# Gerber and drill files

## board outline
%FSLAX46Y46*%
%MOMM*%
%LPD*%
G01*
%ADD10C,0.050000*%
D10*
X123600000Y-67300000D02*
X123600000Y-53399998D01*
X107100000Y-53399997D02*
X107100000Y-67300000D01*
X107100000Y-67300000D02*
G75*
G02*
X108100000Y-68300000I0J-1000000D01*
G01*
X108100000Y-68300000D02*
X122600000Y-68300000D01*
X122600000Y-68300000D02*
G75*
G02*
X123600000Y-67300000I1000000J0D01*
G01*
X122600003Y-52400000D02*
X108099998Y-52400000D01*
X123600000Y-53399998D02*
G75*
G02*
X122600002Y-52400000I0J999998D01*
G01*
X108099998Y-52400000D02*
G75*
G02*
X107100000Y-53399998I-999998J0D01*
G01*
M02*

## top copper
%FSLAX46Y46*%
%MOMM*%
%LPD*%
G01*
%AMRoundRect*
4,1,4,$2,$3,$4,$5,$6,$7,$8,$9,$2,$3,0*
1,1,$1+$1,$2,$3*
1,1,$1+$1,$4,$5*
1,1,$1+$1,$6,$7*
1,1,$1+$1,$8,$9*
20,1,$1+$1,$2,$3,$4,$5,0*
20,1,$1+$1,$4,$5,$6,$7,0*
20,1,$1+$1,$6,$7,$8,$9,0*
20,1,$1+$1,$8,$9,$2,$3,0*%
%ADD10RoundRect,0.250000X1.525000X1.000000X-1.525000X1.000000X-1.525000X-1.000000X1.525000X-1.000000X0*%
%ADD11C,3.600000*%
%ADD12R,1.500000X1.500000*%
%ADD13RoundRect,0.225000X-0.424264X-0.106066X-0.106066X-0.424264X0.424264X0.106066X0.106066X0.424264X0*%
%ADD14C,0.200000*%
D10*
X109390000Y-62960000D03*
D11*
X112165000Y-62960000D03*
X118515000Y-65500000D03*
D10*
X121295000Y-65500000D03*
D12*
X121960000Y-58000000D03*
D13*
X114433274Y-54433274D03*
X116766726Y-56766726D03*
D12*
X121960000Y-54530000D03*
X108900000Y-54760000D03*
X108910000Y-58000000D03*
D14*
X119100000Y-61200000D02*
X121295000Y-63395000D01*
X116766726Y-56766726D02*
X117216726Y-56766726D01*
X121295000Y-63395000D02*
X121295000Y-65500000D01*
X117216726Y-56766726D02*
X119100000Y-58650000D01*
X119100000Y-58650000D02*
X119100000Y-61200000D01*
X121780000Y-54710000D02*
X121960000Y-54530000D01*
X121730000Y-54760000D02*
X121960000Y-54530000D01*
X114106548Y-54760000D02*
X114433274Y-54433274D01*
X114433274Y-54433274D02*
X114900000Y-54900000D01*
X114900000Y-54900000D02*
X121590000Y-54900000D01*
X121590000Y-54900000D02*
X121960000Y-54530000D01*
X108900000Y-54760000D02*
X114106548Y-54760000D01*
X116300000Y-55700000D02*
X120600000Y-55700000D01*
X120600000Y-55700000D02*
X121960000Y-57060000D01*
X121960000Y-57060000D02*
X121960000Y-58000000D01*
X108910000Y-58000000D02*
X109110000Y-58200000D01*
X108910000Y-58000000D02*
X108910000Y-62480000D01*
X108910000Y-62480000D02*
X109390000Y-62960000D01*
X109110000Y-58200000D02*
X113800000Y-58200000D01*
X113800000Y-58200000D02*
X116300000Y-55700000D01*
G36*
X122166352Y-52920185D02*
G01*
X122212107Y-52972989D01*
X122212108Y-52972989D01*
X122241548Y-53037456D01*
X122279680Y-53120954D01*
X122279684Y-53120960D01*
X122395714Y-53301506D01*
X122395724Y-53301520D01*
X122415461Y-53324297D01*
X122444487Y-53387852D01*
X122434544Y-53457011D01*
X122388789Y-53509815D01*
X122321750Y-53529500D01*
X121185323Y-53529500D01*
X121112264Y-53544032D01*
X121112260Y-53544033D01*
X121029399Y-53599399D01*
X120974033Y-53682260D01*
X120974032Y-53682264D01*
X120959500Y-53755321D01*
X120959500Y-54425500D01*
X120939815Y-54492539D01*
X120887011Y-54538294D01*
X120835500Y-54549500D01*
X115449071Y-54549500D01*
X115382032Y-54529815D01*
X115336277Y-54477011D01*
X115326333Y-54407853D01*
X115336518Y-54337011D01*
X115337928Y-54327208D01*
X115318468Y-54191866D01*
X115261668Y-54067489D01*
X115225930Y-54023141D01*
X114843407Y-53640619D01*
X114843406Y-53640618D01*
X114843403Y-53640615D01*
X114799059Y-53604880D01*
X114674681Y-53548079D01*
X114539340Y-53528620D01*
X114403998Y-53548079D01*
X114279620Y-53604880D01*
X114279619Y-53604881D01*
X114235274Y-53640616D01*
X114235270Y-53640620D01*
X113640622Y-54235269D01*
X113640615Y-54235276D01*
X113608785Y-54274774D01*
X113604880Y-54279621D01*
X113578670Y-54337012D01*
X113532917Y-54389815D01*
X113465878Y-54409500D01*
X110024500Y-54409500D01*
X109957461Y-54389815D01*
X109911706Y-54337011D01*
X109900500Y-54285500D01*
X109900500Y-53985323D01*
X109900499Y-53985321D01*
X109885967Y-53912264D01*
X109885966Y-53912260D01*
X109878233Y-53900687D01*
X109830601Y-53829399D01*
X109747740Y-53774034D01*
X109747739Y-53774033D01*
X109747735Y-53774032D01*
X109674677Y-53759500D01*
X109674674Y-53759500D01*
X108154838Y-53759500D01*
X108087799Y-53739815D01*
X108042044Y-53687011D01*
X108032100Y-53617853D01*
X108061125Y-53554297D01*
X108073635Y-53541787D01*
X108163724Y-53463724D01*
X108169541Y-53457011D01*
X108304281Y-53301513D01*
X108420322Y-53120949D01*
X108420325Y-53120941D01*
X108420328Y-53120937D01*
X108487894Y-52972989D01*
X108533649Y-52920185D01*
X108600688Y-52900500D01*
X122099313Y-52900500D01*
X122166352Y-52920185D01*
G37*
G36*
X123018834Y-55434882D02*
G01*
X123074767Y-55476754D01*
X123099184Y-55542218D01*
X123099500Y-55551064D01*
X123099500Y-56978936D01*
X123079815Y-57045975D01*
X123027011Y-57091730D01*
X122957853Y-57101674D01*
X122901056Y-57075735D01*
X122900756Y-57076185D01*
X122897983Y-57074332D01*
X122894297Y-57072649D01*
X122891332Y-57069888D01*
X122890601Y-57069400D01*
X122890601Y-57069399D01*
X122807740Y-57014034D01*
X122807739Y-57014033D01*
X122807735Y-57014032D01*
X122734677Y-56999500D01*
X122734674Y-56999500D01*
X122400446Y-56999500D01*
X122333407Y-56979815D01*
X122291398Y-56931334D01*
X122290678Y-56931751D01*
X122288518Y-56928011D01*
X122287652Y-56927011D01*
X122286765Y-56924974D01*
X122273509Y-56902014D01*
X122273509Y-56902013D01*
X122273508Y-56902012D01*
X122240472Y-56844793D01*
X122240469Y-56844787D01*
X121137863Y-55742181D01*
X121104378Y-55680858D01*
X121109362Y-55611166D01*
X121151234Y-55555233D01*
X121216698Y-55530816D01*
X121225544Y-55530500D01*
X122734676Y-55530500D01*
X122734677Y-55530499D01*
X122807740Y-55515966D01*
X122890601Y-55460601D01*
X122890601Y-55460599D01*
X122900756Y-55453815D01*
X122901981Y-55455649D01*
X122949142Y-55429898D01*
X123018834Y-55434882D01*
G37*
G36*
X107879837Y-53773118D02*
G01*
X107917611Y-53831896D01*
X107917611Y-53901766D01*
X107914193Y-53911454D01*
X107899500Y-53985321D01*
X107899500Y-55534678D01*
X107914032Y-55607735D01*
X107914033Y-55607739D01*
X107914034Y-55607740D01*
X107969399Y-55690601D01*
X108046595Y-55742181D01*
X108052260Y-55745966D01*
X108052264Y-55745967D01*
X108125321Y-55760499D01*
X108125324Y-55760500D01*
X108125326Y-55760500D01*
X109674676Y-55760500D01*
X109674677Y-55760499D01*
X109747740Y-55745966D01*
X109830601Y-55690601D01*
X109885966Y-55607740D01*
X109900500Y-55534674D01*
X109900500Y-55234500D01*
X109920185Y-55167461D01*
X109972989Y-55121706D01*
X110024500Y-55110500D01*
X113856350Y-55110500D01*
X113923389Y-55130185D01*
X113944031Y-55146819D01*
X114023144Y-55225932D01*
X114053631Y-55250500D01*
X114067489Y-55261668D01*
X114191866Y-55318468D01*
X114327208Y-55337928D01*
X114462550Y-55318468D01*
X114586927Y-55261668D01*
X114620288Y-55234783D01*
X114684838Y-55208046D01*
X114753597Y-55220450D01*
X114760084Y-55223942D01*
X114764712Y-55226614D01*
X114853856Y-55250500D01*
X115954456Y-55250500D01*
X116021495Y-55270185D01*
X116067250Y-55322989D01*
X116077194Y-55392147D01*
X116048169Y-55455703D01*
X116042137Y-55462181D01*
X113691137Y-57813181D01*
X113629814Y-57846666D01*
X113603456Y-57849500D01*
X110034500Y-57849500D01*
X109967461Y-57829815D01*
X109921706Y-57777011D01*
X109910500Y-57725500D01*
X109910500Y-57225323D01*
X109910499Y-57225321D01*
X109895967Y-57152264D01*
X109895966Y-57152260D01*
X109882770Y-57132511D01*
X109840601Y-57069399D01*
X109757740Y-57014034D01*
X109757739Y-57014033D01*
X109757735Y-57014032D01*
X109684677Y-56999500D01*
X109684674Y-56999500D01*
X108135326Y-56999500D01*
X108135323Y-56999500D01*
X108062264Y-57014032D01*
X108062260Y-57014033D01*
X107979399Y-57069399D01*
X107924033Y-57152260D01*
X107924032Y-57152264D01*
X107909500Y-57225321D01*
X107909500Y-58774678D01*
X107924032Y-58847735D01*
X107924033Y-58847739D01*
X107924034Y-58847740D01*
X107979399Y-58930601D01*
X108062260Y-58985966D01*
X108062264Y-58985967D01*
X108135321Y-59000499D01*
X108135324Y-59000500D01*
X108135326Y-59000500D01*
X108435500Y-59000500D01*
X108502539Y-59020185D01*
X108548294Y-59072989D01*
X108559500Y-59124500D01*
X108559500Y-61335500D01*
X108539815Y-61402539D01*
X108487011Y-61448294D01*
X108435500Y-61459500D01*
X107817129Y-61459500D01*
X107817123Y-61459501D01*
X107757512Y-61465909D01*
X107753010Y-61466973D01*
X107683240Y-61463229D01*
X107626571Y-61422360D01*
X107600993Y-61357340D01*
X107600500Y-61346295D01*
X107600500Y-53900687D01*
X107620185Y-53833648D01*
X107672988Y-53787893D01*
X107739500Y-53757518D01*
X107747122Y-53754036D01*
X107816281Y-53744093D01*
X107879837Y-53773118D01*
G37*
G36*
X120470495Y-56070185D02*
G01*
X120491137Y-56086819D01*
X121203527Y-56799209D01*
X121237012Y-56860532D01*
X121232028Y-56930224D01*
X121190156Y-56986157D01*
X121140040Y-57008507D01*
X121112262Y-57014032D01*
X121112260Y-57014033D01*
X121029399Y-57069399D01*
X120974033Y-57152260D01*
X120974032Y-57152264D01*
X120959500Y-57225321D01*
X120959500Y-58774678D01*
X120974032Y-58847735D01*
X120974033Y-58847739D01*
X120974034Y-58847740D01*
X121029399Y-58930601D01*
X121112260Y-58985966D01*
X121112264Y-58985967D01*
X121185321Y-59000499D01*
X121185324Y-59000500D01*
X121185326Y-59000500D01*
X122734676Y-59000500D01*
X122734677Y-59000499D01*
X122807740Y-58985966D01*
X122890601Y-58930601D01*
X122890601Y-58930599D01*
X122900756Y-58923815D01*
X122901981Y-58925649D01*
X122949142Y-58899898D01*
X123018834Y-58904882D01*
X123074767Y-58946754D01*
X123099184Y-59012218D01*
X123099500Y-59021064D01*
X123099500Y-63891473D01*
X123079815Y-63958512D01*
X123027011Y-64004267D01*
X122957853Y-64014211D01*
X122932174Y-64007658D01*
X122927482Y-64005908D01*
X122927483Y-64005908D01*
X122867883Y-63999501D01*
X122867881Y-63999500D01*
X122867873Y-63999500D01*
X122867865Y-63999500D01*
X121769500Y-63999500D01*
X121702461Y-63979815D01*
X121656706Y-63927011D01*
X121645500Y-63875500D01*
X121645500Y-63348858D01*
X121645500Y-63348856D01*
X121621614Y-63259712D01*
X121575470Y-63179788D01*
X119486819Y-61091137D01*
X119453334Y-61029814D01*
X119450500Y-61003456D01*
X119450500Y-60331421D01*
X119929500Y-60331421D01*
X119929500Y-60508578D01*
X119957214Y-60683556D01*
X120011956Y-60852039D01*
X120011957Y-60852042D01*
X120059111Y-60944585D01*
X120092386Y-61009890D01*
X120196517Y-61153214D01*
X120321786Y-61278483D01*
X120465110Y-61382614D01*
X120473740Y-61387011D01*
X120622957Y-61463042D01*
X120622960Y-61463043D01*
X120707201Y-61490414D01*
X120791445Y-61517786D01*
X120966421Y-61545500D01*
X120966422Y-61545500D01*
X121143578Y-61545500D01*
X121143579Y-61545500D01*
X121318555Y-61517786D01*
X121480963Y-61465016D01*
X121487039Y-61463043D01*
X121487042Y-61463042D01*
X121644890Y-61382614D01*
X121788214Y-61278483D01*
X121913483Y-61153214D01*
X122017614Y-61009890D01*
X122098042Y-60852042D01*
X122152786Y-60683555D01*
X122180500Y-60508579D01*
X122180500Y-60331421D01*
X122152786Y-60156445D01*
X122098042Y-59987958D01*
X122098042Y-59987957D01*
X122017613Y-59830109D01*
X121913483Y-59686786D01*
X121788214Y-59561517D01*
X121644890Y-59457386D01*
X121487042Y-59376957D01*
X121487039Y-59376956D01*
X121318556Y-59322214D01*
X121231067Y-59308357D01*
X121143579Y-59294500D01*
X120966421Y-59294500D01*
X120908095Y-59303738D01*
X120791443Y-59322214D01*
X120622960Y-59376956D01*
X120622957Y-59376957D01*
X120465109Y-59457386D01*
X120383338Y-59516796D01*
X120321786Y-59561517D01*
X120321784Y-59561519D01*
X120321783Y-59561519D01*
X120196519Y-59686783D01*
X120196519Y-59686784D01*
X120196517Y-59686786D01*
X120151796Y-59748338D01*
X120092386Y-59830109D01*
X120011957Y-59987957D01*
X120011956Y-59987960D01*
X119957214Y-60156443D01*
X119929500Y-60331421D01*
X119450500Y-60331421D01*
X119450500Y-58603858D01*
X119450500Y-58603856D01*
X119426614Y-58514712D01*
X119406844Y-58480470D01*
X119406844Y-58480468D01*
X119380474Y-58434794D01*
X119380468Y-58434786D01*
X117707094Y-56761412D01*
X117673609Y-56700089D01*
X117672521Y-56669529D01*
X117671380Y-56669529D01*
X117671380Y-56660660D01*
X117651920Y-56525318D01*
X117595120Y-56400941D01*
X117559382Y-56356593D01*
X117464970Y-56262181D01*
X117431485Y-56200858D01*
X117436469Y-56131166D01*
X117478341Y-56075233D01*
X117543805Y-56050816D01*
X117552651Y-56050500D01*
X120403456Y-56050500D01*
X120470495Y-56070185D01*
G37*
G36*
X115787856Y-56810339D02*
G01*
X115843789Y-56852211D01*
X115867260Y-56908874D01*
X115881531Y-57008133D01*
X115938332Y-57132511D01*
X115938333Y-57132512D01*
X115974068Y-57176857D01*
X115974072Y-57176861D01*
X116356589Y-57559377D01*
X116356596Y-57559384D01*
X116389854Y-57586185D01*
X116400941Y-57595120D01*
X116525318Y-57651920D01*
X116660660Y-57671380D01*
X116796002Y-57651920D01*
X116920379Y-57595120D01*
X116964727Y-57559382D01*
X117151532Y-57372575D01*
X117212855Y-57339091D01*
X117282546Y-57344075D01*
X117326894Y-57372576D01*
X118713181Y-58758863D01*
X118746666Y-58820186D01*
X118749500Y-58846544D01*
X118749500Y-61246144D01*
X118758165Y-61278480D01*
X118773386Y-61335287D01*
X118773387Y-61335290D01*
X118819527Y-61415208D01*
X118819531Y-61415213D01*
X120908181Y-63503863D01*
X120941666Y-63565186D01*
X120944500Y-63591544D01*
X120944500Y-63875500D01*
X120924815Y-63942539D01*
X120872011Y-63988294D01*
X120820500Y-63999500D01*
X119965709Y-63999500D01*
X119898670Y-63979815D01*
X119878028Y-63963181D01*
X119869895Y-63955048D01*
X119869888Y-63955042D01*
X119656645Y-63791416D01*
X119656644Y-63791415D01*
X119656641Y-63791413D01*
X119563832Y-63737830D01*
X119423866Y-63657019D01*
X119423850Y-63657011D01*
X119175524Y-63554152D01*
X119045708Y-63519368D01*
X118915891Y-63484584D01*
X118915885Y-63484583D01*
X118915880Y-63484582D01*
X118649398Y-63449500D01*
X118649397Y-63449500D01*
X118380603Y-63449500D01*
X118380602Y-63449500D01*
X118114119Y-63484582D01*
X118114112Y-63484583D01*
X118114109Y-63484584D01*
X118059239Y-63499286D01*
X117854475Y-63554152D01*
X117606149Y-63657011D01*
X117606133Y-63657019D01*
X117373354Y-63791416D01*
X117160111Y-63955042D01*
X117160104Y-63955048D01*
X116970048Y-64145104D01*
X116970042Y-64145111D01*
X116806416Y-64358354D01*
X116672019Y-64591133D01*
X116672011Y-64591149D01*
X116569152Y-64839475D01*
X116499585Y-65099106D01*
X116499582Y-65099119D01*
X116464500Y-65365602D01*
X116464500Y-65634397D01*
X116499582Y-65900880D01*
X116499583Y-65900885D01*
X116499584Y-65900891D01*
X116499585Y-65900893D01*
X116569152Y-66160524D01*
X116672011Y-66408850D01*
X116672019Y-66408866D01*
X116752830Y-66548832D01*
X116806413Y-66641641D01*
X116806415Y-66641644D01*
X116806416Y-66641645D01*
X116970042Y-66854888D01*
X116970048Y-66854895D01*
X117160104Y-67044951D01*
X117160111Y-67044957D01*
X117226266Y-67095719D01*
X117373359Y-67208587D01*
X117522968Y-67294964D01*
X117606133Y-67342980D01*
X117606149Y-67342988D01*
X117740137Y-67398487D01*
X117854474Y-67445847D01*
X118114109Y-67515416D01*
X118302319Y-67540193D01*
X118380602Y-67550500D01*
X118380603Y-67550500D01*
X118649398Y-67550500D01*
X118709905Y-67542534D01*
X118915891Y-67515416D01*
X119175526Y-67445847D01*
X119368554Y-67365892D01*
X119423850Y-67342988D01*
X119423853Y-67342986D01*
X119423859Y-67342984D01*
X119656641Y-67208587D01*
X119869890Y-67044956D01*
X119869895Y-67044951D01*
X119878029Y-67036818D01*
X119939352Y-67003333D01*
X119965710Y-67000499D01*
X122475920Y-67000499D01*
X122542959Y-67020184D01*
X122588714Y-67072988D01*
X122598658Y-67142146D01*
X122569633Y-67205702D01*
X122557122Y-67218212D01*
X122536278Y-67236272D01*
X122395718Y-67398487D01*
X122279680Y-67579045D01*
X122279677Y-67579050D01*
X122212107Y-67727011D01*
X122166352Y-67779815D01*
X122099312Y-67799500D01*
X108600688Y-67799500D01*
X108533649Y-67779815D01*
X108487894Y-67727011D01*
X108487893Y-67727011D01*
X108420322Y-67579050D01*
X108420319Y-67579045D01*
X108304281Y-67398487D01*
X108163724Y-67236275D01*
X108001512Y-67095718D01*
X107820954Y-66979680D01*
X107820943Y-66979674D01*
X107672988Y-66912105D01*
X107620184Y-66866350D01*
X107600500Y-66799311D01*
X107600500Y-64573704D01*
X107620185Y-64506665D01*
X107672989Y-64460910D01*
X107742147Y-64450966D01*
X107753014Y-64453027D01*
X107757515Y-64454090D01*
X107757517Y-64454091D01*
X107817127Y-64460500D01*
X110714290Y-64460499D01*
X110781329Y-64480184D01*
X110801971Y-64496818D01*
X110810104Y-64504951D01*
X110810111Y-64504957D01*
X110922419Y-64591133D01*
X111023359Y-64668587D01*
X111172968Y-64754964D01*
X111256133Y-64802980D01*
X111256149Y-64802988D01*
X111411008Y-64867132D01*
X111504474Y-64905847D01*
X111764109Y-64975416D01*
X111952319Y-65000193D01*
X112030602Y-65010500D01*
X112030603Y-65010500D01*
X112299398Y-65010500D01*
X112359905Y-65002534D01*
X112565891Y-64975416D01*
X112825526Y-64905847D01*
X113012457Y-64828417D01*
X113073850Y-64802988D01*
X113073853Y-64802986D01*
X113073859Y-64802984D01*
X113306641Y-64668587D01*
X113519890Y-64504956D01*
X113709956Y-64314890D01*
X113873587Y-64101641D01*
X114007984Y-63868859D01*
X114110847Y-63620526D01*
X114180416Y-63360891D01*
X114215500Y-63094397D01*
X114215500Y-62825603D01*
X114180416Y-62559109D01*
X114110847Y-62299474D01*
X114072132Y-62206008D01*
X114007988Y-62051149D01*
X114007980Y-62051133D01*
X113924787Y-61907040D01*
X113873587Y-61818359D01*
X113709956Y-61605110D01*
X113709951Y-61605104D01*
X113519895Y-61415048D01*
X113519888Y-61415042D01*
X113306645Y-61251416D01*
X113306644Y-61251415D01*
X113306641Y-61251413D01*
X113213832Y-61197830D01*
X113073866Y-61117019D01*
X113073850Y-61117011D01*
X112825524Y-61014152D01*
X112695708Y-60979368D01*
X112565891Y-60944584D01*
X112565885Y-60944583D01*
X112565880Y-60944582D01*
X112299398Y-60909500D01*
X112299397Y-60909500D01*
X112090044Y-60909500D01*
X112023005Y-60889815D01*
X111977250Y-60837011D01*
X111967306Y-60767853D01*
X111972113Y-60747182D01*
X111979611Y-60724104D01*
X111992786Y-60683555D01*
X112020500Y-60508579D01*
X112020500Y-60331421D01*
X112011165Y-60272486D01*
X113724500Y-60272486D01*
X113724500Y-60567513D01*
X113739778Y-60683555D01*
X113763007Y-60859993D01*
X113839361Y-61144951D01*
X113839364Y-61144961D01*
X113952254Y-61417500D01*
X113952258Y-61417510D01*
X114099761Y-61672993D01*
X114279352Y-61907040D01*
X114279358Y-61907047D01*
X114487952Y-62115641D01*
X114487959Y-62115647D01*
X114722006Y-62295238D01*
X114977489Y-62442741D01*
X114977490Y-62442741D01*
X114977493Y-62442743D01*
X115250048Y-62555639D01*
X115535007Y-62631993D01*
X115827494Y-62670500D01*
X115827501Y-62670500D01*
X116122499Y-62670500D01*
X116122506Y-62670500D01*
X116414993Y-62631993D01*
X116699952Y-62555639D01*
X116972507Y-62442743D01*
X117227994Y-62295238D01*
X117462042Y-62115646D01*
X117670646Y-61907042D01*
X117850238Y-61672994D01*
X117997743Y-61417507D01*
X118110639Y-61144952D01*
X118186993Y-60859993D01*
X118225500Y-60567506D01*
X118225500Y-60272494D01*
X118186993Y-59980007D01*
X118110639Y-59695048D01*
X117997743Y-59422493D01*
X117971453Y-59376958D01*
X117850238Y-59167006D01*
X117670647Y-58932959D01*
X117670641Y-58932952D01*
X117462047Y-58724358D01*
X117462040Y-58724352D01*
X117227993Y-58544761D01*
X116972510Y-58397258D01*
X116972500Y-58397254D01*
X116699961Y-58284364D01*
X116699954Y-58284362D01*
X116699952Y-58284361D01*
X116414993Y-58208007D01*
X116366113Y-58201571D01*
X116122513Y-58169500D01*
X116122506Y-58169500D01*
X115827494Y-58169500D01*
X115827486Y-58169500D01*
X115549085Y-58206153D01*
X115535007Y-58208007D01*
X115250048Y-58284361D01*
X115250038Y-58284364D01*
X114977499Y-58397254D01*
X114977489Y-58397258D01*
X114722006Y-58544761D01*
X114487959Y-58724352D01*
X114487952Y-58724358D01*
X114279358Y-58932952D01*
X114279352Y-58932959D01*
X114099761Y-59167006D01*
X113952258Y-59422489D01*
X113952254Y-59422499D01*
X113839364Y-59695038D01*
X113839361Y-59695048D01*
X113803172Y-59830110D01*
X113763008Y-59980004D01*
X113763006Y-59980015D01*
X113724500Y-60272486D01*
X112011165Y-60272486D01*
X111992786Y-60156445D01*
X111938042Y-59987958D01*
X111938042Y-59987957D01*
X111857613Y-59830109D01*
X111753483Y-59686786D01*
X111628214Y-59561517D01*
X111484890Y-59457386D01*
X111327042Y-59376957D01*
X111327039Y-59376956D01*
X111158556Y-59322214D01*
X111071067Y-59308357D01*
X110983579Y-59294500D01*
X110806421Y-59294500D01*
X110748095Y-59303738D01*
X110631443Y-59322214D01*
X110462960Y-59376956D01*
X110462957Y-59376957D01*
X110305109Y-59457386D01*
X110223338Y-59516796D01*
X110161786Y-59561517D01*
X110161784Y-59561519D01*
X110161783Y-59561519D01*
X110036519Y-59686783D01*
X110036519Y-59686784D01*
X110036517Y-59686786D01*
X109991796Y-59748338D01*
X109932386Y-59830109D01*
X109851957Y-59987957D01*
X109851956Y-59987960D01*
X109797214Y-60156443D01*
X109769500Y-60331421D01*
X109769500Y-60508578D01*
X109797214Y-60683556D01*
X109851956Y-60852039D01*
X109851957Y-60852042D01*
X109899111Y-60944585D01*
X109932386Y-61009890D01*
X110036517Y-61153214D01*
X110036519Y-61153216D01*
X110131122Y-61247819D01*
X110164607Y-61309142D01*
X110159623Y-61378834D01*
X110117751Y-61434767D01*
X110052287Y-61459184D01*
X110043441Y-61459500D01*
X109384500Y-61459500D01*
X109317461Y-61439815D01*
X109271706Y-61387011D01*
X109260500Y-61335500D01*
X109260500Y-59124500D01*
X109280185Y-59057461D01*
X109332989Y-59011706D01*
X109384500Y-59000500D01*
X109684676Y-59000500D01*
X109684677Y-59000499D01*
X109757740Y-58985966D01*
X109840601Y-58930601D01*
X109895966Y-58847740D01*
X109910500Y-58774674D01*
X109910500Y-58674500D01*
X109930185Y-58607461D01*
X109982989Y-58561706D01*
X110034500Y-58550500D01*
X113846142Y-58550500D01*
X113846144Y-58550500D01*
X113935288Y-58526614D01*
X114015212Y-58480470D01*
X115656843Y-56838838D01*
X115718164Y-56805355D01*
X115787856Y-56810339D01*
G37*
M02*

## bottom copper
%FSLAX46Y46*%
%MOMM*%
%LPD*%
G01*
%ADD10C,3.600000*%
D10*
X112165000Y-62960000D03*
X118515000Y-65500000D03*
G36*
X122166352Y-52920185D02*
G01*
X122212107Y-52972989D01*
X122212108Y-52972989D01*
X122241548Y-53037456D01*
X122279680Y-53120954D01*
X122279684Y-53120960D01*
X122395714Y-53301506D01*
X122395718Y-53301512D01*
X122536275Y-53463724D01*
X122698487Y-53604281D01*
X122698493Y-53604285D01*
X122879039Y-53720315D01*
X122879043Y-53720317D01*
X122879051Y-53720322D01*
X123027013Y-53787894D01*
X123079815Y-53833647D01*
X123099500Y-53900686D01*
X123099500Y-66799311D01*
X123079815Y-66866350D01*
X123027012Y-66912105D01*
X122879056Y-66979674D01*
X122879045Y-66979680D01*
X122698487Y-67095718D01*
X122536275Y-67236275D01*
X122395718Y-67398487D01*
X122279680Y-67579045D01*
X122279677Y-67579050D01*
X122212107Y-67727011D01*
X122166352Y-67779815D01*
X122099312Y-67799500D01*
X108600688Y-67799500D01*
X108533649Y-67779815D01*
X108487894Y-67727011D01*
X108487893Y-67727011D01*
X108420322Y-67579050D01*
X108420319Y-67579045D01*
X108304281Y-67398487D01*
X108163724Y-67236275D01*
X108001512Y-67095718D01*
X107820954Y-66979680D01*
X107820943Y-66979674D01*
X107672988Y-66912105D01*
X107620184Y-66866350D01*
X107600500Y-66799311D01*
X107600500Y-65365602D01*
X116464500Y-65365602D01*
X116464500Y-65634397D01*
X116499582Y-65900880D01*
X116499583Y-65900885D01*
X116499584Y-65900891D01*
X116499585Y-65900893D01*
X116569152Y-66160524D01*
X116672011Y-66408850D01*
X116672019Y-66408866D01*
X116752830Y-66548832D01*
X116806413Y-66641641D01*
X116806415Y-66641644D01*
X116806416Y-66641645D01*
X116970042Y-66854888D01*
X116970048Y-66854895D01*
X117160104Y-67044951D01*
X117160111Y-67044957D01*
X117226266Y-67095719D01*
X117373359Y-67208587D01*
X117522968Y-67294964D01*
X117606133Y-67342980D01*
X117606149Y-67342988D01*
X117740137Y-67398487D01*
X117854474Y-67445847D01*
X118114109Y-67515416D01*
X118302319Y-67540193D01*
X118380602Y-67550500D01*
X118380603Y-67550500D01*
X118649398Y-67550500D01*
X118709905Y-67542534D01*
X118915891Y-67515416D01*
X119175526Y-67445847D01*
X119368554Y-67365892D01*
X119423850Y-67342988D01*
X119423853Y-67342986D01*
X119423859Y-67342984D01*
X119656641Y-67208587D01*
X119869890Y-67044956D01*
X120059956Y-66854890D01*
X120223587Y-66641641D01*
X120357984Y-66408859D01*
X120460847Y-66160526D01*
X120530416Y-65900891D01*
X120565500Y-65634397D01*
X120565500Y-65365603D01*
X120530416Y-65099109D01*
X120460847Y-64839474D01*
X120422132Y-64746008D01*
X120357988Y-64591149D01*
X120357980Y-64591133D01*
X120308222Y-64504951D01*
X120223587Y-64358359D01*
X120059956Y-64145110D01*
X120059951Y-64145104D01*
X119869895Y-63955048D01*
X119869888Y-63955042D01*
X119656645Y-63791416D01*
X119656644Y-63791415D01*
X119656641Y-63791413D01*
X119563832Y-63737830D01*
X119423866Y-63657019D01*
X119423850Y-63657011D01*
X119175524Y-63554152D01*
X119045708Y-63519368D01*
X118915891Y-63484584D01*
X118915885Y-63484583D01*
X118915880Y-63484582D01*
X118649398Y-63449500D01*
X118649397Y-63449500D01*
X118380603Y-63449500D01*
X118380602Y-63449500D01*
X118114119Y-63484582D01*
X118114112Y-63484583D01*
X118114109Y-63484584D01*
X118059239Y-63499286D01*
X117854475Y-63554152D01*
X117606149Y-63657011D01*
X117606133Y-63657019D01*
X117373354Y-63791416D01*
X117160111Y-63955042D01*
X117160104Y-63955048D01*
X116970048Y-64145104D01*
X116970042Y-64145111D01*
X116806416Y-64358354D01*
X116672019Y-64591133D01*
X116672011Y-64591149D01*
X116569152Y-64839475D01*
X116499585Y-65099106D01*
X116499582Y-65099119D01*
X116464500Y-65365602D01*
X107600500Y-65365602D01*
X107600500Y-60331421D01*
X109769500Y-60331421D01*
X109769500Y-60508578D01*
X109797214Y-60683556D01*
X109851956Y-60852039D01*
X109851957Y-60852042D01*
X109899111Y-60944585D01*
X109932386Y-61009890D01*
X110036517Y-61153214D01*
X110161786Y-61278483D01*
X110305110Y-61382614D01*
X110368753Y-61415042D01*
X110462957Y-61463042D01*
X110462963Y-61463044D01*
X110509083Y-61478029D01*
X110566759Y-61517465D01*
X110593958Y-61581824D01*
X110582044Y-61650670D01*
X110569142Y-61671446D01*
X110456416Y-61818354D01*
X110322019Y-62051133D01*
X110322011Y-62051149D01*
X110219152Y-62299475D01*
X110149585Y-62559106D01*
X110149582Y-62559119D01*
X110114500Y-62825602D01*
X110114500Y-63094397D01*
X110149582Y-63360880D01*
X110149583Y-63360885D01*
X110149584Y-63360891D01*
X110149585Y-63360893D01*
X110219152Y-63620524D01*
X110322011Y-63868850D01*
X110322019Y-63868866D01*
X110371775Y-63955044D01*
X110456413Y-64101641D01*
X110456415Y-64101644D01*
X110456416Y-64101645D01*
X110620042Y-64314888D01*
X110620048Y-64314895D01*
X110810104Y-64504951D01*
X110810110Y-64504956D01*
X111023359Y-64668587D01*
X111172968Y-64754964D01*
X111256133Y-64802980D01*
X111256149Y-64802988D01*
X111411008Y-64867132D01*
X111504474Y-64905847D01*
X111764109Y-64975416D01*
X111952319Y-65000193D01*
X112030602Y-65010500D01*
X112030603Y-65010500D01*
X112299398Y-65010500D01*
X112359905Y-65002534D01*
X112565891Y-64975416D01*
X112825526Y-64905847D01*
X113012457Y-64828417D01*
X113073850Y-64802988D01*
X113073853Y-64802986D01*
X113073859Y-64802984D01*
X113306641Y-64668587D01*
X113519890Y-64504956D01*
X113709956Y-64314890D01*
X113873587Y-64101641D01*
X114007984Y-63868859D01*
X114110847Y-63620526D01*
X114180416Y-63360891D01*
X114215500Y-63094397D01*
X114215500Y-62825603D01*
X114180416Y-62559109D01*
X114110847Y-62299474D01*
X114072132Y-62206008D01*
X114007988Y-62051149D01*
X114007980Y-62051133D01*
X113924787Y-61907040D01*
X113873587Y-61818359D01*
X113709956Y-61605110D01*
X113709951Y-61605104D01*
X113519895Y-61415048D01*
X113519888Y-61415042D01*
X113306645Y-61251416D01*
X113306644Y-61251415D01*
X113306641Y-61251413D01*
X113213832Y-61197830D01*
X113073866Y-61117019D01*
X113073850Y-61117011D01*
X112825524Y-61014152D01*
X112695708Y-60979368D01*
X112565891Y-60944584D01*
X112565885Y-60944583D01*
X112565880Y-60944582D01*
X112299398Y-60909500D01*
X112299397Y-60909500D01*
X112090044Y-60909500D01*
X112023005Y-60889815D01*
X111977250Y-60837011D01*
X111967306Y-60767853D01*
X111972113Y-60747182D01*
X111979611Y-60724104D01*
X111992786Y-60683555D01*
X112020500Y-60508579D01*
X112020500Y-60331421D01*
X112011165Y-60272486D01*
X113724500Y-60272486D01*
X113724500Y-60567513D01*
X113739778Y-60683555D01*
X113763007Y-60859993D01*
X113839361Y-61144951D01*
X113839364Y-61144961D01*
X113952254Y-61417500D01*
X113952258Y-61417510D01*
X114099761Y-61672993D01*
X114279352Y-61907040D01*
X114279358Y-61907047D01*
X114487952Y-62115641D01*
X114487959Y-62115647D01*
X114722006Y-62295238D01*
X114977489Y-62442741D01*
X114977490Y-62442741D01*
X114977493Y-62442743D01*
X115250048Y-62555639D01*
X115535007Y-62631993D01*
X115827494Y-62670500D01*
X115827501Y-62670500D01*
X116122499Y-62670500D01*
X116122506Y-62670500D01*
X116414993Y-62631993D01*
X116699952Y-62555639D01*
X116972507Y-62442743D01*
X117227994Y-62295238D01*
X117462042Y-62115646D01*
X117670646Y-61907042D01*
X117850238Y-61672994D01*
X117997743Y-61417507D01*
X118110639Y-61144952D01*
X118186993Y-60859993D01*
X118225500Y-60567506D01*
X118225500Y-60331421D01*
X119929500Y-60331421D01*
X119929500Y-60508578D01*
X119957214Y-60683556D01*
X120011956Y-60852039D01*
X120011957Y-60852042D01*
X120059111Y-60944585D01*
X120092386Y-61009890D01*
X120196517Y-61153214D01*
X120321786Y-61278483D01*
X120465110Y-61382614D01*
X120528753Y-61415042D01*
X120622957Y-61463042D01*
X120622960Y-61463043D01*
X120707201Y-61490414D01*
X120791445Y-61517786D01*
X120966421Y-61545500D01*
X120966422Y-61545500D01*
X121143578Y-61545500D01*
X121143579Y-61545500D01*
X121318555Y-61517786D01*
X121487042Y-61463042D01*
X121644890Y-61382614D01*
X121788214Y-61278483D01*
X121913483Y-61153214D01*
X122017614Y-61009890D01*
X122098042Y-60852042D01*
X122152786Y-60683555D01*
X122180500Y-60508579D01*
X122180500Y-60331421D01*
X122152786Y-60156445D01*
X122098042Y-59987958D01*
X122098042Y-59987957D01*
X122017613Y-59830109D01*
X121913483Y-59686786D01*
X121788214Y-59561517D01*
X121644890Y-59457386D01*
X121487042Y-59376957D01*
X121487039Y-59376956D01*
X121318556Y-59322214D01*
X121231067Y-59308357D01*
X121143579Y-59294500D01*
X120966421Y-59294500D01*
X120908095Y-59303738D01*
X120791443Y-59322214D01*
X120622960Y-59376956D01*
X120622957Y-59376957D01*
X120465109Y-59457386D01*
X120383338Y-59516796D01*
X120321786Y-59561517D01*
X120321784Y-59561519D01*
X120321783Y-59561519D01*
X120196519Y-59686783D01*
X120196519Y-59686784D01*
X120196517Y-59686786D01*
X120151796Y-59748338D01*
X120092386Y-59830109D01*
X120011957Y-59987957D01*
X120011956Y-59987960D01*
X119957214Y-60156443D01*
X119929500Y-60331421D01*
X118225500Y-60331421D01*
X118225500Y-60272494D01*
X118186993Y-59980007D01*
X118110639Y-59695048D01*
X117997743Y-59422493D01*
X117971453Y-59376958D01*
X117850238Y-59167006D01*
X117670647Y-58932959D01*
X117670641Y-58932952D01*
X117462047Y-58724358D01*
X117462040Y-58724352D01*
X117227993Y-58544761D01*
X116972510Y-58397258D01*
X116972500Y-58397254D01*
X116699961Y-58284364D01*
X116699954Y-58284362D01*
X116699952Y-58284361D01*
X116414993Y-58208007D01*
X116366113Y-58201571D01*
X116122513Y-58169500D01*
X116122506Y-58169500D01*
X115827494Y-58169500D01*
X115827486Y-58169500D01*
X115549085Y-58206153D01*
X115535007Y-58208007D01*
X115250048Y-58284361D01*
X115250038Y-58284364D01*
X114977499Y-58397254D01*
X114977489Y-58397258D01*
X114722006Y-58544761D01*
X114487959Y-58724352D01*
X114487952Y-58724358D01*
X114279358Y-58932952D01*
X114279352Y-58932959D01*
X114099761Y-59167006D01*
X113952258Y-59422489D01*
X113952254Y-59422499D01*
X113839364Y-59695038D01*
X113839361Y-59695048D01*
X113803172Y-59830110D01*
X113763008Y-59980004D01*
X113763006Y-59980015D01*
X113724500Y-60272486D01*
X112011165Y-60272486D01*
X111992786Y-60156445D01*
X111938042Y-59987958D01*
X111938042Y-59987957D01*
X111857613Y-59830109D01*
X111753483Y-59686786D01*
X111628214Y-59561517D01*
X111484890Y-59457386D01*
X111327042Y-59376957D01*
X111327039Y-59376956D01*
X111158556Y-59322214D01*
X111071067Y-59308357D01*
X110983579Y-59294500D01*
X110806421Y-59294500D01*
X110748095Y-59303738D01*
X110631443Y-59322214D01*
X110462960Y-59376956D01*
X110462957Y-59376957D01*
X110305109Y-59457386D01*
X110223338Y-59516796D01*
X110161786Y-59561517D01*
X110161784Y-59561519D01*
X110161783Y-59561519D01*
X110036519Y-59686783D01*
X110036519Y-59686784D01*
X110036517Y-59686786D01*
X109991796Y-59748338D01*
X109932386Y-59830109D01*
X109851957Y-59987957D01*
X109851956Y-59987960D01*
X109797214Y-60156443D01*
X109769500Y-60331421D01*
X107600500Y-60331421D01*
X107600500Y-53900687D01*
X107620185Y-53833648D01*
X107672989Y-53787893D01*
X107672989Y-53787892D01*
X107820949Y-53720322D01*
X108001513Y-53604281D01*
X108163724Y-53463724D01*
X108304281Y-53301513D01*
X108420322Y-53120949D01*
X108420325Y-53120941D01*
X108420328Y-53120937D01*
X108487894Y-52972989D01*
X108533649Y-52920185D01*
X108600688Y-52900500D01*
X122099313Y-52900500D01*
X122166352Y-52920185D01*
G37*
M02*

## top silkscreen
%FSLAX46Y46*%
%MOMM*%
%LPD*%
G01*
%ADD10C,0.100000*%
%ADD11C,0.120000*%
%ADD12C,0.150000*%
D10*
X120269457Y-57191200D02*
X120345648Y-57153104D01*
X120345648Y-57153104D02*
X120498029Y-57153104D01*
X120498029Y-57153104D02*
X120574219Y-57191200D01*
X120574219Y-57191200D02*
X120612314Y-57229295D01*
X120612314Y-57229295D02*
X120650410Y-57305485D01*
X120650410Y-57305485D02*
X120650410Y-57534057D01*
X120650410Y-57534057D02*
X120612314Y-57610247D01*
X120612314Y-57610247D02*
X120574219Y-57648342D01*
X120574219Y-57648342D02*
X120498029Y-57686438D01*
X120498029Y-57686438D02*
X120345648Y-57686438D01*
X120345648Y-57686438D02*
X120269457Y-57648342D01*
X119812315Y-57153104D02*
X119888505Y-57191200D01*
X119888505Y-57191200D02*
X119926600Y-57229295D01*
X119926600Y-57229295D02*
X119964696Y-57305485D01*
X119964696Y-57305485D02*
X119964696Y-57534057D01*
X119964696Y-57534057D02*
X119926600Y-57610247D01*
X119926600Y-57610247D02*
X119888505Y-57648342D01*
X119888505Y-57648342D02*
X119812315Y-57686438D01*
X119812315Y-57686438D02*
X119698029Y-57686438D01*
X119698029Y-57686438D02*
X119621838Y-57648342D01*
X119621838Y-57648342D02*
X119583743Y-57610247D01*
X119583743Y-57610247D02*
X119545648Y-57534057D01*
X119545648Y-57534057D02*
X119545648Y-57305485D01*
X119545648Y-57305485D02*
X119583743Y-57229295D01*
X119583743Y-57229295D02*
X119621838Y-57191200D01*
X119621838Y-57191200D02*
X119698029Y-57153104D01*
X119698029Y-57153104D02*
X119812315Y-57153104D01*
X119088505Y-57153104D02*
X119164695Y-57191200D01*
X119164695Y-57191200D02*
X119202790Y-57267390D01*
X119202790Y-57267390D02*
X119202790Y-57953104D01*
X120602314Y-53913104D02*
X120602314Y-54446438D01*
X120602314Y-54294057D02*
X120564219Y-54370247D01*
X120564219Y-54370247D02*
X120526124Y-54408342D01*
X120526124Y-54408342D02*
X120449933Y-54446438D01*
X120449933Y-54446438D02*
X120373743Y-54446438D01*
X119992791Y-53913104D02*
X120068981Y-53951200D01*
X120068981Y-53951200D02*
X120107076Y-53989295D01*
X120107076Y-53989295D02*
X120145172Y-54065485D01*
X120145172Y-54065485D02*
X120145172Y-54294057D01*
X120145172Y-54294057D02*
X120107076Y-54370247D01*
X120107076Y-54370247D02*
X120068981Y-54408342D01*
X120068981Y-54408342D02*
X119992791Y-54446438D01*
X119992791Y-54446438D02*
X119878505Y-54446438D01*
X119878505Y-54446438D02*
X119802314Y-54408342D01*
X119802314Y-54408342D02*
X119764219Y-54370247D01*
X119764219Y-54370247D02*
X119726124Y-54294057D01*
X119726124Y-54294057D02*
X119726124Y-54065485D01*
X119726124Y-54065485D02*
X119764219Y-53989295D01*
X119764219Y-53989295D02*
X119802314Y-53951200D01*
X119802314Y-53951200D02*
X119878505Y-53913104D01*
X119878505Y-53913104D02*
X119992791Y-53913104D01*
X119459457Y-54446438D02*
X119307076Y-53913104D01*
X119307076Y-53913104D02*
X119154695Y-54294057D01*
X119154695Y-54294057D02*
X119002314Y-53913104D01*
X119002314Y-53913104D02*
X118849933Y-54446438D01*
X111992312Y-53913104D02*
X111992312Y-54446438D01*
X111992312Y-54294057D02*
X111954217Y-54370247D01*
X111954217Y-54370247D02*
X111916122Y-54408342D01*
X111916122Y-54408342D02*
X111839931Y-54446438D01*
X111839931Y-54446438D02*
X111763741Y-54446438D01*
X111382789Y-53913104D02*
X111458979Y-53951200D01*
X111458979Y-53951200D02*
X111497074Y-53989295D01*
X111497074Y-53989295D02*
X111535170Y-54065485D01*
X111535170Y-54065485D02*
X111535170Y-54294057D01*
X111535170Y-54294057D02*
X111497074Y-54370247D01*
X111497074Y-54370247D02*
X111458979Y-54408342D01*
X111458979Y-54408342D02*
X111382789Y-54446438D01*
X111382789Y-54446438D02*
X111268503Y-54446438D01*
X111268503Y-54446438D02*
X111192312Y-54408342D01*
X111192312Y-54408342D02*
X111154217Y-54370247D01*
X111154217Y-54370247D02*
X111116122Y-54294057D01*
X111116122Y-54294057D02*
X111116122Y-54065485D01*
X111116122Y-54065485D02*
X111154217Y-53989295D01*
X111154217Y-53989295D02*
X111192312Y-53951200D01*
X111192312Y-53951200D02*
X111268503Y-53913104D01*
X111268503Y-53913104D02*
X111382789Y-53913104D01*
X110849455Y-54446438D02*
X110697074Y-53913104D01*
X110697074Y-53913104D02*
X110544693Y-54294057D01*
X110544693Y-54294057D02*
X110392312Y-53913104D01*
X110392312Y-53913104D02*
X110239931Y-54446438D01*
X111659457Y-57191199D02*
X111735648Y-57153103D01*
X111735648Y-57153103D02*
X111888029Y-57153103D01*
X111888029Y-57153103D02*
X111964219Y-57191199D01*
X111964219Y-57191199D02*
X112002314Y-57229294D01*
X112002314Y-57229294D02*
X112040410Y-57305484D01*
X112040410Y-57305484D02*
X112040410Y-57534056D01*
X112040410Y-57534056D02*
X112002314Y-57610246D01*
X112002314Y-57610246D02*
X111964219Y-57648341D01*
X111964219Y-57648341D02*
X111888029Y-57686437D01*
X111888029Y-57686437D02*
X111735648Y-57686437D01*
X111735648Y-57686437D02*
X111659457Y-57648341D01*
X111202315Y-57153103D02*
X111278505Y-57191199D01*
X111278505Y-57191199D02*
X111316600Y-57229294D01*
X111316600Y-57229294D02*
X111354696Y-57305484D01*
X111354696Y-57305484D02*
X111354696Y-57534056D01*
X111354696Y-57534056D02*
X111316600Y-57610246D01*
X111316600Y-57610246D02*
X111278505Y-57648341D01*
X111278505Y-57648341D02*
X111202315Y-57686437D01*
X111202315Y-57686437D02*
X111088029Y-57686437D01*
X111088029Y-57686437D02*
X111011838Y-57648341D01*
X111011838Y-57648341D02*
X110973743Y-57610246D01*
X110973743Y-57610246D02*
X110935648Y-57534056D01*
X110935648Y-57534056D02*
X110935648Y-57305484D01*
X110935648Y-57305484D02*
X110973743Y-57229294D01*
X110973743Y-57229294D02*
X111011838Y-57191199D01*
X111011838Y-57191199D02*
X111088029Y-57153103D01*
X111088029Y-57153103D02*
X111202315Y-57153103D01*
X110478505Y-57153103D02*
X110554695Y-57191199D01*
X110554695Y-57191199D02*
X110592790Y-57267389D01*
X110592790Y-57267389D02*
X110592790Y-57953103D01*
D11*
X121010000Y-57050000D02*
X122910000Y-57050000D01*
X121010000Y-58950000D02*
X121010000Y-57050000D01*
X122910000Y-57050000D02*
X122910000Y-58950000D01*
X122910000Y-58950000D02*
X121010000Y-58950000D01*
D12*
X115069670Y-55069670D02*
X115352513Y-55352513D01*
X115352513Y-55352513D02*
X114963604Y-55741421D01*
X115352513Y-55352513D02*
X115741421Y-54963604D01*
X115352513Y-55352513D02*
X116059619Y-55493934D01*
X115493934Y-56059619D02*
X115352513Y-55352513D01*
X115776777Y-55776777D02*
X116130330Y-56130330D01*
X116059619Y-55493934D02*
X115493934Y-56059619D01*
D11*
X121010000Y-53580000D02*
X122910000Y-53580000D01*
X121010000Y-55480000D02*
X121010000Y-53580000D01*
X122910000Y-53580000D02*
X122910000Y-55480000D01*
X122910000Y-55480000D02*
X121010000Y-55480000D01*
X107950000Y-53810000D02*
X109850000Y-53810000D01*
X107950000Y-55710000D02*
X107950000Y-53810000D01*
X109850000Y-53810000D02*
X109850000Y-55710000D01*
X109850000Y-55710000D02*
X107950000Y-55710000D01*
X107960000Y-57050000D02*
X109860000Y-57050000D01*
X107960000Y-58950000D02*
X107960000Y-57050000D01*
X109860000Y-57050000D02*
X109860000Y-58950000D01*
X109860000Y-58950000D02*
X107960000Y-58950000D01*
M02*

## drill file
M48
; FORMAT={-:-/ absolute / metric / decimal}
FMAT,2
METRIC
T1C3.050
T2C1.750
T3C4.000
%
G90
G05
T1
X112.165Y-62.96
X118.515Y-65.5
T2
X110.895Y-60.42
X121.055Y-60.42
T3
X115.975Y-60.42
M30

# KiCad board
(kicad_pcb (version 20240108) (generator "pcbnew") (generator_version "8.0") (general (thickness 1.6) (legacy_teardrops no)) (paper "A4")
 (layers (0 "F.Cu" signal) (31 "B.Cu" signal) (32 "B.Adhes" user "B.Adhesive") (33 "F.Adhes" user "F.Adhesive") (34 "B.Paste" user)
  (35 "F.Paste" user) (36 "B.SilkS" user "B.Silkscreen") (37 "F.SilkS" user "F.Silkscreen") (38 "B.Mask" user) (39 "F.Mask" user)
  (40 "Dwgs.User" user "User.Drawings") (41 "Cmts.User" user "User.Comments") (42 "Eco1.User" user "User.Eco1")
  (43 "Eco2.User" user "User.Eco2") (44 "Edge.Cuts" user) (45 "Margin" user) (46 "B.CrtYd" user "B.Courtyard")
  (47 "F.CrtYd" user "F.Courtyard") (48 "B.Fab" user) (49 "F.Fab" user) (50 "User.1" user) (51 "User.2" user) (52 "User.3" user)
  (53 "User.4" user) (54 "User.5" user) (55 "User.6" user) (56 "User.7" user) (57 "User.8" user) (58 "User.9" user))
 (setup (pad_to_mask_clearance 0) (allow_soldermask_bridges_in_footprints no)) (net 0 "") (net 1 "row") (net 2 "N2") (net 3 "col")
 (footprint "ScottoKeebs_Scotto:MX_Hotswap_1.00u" (layer "F.Cu") (at 115.34 64.23)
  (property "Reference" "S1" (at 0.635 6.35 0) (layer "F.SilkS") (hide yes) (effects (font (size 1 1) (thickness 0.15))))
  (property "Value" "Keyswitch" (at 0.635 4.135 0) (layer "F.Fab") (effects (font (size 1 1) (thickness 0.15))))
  (pad "" smd roundrect (at -6.45 -1.27 180) (size 2.55 2.5) (layers "F.Paste" "F.Mask") (roundrect_rratio 0.1))
  (pad "" np_thru_hole circle (at -4.445 -3.81 180) (size 1.75 1.75) (drill 1.75) (layers "F&B.Cu" "*.Mask") (clearance 0.1))
  (pad "" np_thru_hole circle (at 0.635 -3.81 180) (size 4 4) (drill 4) (layers "*.Cu" "*.Mask"))
  (pad "" np_thru_hole circle (at 5.715 -3.81 180) (size 1.75 1.75) (drill 1.75) (layers "*.Cu" "*.Mask"))
  (pad "" smd roundrect (at 6.477 1.27 180) (size 2.55 2.5) (layers "F.Paste" "F.Mask") (roundrect_rratio 0.1))
  (pad "1" smd roundrect (at -5.95 -1.27 180) (size 3.55 2.5) (layers "F.Cu") (roundrect_rratio 0.1) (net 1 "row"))
  (pad "1" thru_hole circle (at -3.175 -1.27 180) (size 3.6 3.6) (drill 3.05) (layers "*.Cu" "*.Mask") (remove_unused_layers no)
   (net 1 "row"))
  (pad "2" thru_hole circle (at 3.175 1.27 180) (size 3.6 3.6) (drill 3.05) (layers "*.Cu" "*.Mask") (remove_unused_layers no) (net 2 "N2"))
  (pad "2" smd roundrect (at 5.955 1.27 180) (size 3.55 2.5) (layers "F.Cu") (roundrect_rratio 0.1) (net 2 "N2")))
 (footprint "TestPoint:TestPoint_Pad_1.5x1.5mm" (layer "F.Cu") (at 121.96 58)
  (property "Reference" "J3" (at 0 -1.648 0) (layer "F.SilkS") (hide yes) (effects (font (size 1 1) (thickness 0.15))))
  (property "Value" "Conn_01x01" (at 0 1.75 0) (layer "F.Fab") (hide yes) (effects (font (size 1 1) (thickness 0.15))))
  (fp_line (start -0.95 -0.95) (end 0.95 -0.95) (stroke (width 0.12) (type solid)) (layer "F.SilkS"))
  (fp_line (start -0.95 0.95) (end -0.95 -0.95) (stroke (width 0.12) (type solid)) (layer "F.SilkS"))
  (fp_line (start 0.95 -0.95) (end 0.95 0.95) (stroke (width 0.12) (type solid)) (layer "F.SilkS"))
  (fp_line (start 0.95 0.95) (end -0.95 0.95) (stroke (width 0.12) (type solid)) (layer "F.SilkS"))
  (pad "1" smd rect (at 0 0) (size 1.5 1.5) (layers "F.Cu" "F.Mask") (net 1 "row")))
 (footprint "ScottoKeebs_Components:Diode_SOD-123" (layer "F.Cu") (at 115.6 55.6 -45)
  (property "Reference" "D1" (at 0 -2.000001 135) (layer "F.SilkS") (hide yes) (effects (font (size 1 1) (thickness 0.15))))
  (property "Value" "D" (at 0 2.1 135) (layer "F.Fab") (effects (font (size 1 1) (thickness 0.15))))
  (fp_line (start -0.75 0) (end -0.349999 0) (stroke (width 0.15) (type solid)) (layer "F.SilkS"))
  (fp_line (start -0.349999 0) (end -0.35 0.55) (stroke (width 0.15) (type solid)) (layer "F.SilkS"))
  (fp_line (start -0.349999 0) (end -0.35 -0.55) (stroke (width 0.15) (type solid)) (layer "F.SilkS"))
  (fp_line (start -0.349999 0) (end 0.25 -0.4) (stroke (width 0.15) (type solid)) (layer "F.SilkS"))
  (fp_line (start 0.25 0.4) (end -0.349999 0) (stroke (width 0.15) (type solid)) (layer "F.SilkS"))
  (fp_line (start 0.25 0) (end 0.75 0) (stroke (width 0.15) (type solid)) (layer "F.SilkS"))
  (fp_line (start 0.25 -0.4) (end 0.25 0.4) (stroke (width 0.15) (type solid)) (layer "F.SilkS"))
  (pad "1" smd roundrect (at -1.65 0 315) (size 0.9 1.2) (layers "F.Cu" "F.Paste" "F.Mask") (roundrect_rratio 0.25) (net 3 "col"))
  (pad "2" smd roundrect (at 1.65 0 315) (size 0.9 1.2) (layers "F.Cu" "F.Paste" "F.Mask") (roundrect_rratio 0.25) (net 2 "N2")))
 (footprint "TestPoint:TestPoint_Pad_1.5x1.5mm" (layer "F.Cu") (at 121.96 54.53)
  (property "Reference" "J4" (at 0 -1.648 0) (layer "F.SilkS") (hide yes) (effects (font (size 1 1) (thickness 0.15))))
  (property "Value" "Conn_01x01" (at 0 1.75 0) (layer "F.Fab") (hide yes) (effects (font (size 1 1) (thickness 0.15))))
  (fp_line (start -0.95 -0.95) (end 0.95 -0.95) (stroke (width 0.12) (type solid)) (layer "F.SilkS"))
  (fp_line (start -0.95 0.95) (end -0.95 -0.95) (stroke (width 0.12) (type solid)) (layer "F.SilkS"))
  (fp_line (start 0.95 -0.95) (end 0.95 0.95) (stroke (width 0.12) (type solid)) (layer "F.SilkS"))
  (fp_line (start 0.95 0.95) (end -0.95 0.95) (stroke (width 0.12) (type solid)) (layer "F.SilkS"))
  (pad "1" smd rect (at 0 0) (size 1.5 1.5) (layers "F.Cu" "F.Mask") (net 3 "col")))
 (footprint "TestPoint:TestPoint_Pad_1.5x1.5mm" (layer "F.Cu") (at 108.9 54.76)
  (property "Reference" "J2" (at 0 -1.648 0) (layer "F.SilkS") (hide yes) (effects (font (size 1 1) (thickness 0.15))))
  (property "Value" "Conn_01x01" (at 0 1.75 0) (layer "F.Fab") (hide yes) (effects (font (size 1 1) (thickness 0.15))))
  (fp_line (start -0.95 -0.95) (end 0.95 -0.95) (stroke (width 0.12) (type solid)) (layer "F.SilkS"))
  (fp_line (start -0.95 0.95) (end -0.95 -0.95) (stroke (width 0.12) (type solid)) (layer "F.SilkS"))
  (fp_line (start 0.95 -0.95) (end 0.95 0.95) (stroke (width 0.12) (type solid)) (layer "F.SilkS"))
  (fp_line (start 0.95 0.95) (end -0.95 0.95) (stroke (width 0.12) (type solid)) (layer "F.SilkS"))
  (pad "1" smd rect (at 0 0) (size 1.5 1.5) (layers "F.Cu" "F.Mask") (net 3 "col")))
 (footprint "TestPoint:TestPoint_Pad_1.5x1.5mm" (layer "F.Cu") (at 108.91 58)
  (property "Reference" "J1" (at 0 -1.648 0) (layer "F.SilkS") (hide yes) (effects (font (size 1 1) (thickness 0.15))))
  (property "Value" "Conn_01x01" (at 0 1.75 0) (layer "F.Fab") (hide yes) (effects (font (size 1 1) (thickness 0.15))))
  (fp_line (start -0.95 -0.95) (end 0.95 -0.95) (stroke (width 0.12) (type solid)) (layer "F.SilkS"))
  (fp_line (start -0.95 0.95) (end -0.95 -0.95) (stroke (width 0.12) (type solid)) (layer "F.SilkS"))
  (fp_line (start 0.95 -0.95) (end 0.95 0.95) (stroke (width 0.12) (type solid)) (layer "F.SilkS"))
  (fp_line (start 0.95 0.95) (end -0.95 0.95) (stroke (width 0.12) (type solid)) (layer "F.SilkS"))
  (pad "1" smd rect (at 0 0) (size 1.5 1.5) (layers "F.Cu" "F.Mask") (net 1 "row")))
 (gr_line (start 123.6 67.3) (end 123.6 53.399998) (stroke (width 0.05) (type default)) (layer "Edge.Cuts"))
 (gr_line (start 107.1 53.399997) (end 107.1 67.3) (stroke (width 0.05) (type default)) (layer "Edge.Cuts"))
 (gr_arc (start 107.1 67.3) (mid 107.807107 67.592893) (end 108.1 68.3) (stroke (width 0.05) (type default)) (layer "Edge.Cuts"))
 (gr_line (start 108.1 68.3) (end 122.6 68.3) (stroke (width 0.05) (type default)) (layer "Edge.Cuts"))
 (gr_arc (start 122.6 68.3) (mid 122.892893 67.592893) (end 123.6 67.3) (stroke (width 0.05) (type default)) (layer "Edge.Cuts"))
 (gr_line (start 122.600003 52.4) (end 108.099998 52.4) (stroke (width 0.05) (type default)) (layer "Edge.Cuts"))
 (gr_arc (start 123.6 53.399998) (mid 122.892893 53.107107) (end 122.600003 52.4) (stroke (width 0.05) (type default)) (layer "Edge.Cuts"))
 (gr_arc (start 108.099998 52.4) (mid 107.807107 53.107107) (end 107.1 53.399997) (stroke (width 0.05) (type default)) (layer "Edge.Cuts"))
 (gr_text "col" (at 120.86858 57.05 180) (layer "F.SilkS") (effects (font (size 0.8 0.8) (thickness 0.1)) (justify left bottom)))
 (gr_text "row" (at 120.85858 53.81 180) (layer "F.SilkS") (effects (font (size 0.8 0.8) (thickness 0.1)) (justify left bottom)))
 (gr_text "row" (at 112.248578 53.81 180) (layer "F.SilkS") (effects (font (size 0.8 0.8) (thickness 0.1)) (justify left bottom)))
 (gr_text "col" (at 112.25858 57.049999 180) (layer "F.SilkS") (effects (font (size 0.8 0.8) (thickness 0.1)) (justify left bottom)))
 (segment (start 119.1 61.2) (end 121.295 63.395) (width 0.2) (layer "F.Cu") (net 2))
 (segment (start 116.766726 56.766726) (end 117.216726 56.766726) (width 0.2) (layer "F.Cu") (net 2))
 (segment (start 121.295 63.395) (end 121.295 65.5) (width 0.2) (layer "F.Cu") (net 2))
 (segment (start 117.216726 56.766726) (end 119.1 58.65) (width 0.2) (layer "F.Cu") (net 2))
 (segment (start 119.1 58.65) (end 119.1 61.2) (width 0.2) (layer "F.Cu") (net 2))
 (segment (start 121.78 54.71) (end 121.96 54.53) (width 0.2) (layer "F.Cu") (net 3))
 (segment (start 121.73 54.76) (end 121.96 54.53) (width 0.2) (layer "F.Cu") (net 3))
 (segment (start 114.106548 54.76) (end 114.433274 54.433274) (width 0.2) (layer "F.Cu") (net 3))
 (segment (start 114.433274 54.433274) (end 114.9 54.9) (width 0.2) (layer "F.Cu") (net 3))
 (segment (start 114.9 54.9) (end 121.59 54.9) (width 0.2) (layer "F.Cu") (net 3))
 (segment (start 121.59 54.9) (end 121.96 54.53) (width 0.2) (layer "F.Cu") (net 3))
 (segment (start 108.9 54.76) (end 114.106548 54.76) (width 0.2) (layer "F.Cu") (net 3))
 (segment (start 116.3 55.7) (end 120.6 55.7) (width 0.2) (layer "F.Cu") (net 1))
 (segment (start 120.6 55.7) (end 121.96 57.06) (width 0.2) (layer "F.Cu") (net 1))
 (segment (start 121.96 57.06) (end 121.96 58) (width 0.2) (layer "F.Cu") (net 1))
 (segment (start 108.91 58) (end 109.11 58.2) (width 0.2) (layer "F.Cu") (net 1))
 (segment (start 108.91 58) (end 108.91 62.48) (width 0.2) (layer "F.Cu") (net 1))
 (segment (start 108.91 62.48) (end 109.39 62.96) (width 0.2) (layer "F.Cu") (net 1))
 (segment (start 109.11 58.2) (end 113.8 58.2) (width 0.2) (layer "F.Cu") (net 1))
 (segment (start 113.8 58.2) (end 116.3 55.7) (width 0.2) (layer "F.Cu") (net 1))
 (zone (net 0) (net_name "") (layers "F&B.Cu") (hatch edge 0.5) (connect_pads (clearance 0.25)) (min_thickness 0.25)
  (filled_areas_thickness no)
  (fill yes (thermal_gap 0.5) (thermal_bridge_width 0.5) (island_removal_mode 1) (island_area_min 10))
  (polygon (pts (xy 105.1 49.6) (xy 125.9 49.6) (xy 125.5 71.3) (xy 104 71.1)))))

